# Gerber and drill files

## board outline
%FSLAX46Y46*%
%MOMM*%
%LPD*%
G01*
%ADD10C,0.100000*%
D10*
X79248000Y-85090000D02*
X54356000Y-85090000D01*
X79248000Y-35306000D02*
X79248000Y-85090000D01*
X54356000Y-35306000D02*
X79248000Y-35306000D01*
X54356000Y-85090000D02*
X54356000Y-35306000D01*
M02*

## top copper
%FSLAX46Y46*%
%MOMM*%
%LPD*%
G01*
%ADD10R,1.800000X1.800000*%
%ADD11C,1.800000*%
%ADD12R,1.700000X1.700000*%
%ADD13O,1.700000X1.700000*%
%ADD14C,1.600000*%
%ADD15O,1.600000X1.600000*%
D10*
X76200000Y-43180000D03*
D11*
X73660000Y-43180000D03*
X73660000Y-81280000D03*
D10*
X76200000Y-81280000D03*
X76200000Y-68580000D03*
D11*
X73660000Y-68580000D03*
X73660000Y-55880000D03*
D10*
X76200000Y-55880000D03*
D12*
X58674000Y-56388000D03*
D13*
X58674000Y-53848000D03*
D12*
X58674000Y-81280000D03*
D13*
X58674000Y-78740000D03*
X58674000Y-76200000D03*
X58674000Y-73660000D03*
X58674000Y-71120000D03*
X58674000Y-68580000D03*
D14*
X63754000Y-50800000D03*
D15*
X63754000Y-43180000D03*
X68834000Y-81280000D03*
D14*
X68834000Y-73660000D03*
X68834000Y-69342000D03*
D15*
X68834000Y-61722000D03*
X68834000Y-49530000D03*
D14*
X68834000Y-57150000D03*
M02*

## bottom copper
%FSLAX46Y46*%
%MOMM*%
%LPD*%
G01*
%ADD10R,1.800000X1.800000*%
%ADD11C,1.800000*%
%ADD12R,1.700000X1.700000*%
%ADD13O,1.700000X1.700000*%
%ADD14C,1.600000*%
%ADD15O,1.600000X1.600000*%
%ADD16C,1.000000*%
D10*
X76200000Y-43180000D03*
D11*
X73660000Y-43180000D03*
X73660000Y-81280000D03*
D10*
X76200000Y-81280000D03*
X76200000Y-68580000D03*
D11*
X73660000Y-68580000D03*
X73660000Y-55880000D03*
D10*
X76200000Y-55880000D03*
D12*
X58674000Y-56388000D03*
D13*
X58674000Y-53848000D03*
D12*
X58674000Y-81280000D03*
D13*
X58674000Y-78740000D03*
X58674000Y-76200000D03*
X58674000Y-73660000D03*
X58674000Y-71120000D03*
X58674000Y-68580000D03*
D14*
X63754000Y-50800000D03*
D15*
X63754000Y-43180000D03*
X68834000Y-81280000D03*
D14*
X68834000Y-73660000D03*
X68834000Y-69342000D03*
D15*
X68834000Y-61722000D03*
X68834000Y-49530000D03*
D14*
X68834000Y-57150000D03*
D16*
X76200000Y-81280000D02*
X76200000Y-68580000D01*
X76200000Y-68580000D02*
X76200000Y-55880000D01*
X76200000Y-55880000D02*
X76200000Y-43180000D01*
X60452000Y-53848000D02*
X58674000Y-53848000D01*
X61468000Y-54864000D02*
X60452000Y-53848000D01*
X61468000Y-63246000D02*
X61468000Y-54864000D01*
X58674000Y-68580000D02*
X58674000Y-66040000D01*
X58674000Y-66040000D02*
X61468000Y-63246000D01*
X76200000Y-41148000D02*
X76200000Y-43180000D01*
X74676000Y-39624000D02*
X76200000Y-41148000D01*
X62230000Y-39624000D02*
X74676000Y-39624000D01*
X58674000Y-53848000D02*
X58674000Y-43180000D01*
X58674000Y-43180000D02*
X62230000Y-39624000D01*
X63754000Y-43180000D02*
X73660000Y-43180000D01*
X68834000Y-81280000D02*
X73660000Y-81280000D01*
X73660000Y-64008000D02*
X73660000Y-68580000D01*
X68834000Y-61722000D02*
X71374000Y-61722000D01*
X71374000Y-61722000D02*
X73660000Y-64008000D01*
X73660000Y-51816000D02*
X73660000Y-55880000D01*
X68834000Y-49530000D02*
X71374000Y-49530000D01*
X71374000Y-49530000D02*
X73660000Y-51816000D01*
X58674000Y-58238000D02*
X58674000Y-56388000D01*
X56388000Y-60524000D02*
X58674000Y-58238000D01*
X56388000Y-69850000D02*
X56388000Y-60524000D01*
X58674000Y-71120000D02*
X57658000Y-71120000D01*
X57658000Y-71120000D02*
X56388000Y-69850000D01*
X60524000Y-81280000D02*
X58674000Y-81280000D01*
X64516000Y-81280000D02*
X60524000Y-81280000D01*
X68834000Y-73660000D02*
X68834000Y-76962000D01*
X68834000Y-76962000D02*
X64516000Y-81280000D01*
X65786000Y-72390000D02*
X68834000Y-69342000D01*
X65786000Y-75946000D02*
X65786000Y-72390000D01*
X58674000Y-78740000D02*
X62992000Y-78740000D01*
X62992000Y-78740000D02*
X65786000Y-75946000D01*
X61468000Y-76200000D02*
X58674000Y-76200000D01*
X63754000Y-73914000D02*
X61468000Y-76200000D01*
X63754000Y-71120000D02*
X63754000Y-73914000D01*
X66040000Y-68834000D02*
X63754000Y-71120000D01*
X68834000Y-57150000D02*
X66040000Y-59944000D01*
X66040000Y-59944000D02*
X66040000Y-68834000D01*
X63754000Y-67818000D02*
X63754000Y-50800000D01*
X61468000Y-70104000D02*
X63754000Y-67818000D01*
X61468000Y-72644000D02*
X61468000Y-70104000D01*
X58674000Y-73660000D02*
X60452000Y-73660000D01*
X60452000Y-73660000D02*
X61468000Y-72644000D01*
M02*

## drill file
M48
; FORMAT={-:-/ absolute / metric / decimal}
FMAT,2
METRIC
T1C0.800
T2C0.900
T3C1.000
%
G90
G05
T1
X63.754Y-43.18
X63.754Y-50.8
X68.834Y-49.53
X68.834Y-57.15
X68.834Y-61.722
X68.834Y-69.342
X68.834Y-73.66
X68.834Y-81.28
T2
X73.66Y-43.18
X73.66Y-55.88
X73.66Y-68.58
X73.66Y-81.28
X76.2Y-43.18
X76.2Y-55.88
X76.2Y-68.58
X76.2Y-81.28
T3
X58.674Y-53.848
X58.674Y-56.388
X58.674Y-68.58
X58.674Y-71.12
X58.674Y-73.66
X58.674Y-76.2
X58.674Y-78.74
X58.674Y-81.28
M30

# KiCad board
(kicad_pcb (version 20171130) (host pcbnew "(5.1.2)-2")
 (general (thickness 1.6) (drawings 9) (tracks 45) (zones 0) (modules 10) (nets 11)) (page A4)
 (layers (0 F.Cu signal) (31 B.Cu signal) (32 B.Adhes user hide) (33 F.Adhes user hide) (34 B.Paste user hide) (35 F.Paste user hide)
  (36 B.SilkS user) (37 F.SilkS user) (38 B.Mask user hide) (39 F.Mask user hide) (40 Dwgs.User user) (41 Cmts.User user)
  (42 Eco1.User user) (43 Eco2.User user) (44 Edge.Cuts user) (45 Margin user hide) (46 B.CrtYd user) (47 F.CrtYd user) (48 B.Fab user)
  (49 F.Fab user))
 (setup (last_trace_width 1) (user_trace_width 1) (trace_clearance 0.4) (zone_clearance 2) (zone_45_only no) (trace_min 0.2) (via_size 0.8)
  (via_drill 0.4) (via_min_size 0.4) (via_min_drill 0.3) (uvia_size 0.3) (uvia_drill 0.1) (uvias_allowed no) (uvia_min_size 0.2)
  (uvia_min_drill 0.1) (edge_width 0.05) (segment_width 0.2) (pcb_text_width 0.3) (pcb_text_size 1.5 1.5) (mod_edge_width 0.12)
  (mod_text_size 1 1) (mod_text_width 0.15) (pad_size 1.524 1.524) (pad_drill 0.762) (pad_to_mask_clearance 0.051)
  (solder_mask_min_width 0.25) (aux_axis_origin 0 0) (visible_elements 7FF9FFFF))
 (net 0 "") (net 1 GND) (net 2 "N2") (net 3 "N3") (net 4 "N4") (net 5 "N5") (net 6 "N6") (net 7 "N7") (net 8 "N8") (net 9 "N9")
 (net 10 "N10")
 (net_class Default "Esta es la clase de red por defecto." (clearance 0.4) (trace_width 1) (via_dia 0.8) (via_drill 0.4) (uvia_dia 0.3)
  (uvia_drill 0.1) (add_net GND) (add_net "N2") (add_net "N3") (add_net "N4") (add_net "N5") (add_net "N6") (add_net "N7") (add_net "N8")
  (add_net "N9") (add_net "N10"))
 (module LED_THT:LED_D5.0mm (layer F.Cu) (at 76.2 43.18 180)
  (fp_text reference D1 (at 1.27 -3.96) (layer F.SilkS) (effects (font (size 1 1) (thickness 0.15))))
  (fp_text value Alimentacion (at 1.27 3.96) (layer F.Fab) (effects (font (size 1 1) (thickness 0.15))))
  (pad 1 thru_hole rect (at 0 0 180) (size 1.8 1.8) (drill 0.9) (layers *.Cu *.Mask) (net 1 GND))
  (pad 2 thru_hole circle (at 2.54 0 180) (size 1.8 1.8) (drill 0.9) (layers *.Cu *.Mask) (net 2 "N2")))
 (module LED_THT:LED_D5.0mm (layer F.Cu) (at 76.2 81.28 180)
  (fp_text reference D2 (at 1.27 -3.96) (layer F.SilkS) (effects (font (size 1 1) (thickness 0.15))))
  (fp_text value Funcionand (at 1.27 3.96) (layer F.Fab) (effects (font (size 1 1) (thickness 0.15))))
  (pad 2 thru_hole circle (at 2.54 0 180) (size 1.8 1.8) (drill 0.9) (layers *.Cu *.Mask) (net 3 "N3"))
  (pad 1 thru_hole rect (at 0 0 180) (size 1.8 1.8) (drill 0.9) (layers *.Cu *.Mask) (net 1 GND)))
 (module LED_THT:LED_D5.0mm (layer F.Cu) (at 76.2 68.58 180)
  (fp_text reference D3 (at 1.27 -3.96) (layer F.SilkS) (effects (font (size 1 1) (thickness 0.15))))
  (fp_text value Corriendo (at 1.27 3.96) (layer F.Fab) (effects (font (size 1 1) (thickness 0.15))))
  (pad 1 thru_hole rect (at 0 0 180) (size 1.8 1.8) (drill 0.9) (layers *.Cu *.Mask) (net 1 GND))
  (pad 2 thru_hole circle (at 2.54 0 180) (size 1.8 1.8) (drill 0.9) (layers *.Cu *.Mask) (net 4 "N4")))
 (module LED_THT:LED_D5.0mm (layer F.Cu) (at 76.2 55.88 180)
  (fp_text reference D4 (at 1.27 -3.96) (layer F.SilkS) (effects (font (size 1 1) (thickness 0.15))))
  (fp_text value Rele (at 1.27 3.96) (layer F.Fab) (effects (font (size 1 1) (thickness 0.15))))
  (pad 2 thru_hole circle (at 2.54 0 180) (size 1.8 1.8) (drill 0.9) (layers *.Cu *.Mask) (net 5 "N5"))
  (pad 1 thru_hole rect (at 0 0 180) (size 1.8 1.8) (drill 0.9) (layers *.Cu *.Mask) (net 1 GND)))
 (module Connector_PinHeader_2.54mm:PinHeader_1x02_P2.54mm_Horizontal (layer F.Cu) (at 58.674 56.388 180)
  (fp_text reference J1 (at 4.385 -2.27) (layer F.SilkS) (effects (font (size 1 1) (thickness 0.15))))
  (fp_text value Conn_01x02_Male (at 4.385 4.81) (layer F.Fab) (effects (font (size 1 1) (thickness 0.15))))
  (pad 1 thru_hole rect (at 0 0 180) (size 1.7 1.7) (drill 1) (layers *.Cu *.Mask) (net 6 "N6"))
  (pad 2 thru_hole oval (at 0 2.54 180) (size 1.7 1.7) (drill 1) (layers *.Cu *.Mask) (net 1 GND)))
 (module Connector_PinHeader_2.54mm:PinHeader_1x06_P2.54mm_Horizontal (layer F.Cu) (at 58.674 81.28 180)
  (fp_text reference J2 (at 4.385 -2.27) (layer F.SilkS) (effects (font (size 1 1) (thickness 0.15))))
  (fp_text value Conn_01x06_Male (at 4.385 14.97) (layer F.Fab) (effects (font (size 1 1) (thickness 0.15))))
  (pad 1 thru_hole rect (at 0 0 180) (size 1.7 1.7) (drill 1) (layers *.Cu *.Mask) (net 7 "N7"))
  (pad 2 thru_hole oval (at 0 2.54 180) (size 1.7 1.7) (drill 1) (layers *.Cu *.Mask) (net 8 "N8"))
  (pad 3 thru_hole oval (at 0 5.08 180) (size 1.7 1.7) (drill 1) (layers *.Cu *.Mask) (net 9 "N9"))
  (pad 4 thru_hole oval (at 0 7.62 180) (size 1.7 1.7) (drill 1) (layers *.Cu *.Mask) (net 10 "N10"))
  (pad 5 thru_hole oval (at 0 10.16 180) (size 1.7 1.7) (drill 1) (layers *.Cu *.Mask) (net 6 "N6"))
  (pad 6 thru_hole oval (at 0 12.7 180) (size 1.7 1.7) (drill 1) (layers *.Cu *.Mask) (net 1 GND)))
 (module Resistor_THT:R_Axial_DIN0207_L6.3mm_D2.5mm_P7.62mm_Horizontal (layer F.Cu) (at 63.754 50.8 90)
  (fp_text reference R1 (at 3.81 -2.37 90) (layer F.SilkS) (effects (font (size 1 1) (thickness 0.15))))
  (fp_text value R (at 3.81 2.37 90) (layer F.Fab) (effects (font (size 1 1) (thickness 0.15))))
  (pad 1 thru_hole circle (at 0 0 90) (size 1.6 1.6) (drill 0.8) (layers *.Cu *.Mask) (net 10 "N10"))
  (pad 2 thru_hole oval (at 7.62 0 90) (size 1.6 1.6) (drill 0.8) (layers *.Cu *.Mask) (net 2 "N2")))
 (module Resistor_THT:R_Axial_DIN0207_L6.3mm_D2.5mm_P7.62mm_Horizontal (layer F.Cu) (at 68.834 73.66 270)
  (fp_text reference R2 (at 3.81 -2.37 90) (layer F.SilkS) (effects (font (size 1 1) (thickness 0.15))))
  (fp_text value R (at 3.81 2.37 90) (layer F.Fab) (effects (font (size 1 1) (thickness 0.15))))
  (pad 2 thru_hole oval (at 7.62 0 270) (size 1.6 1.6) (drill 0.8) (layers *.Cu *.Mask) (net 3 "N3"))
  (pad 1 thru_hole circle (at 0 0 270) (size 1.6 1.6) (drill 0.8) (layers *.Cu *.Mask) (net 7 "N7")))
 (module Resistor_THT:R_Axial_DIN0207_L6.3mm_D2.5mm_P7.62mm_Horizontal (layer F.Cu) (at 68.834 69.342 90)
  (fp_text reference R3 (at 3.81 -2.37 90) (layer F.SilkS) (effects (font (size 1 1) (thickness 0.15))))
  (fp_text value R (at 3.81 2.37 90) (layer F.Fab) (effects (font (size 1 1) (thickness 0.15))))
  (pad 1 thru_hole circle (at 0 0 90) (size 1.6 1.6) (drill 0.8) (layers *.Cu *.Mask) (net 8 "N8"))
  (pad 2 thru_hole oval (at 7.62 0 90) (size 1.6 1.6) (drill 0.8) (layers *.Cu *.Mask) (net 4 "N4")))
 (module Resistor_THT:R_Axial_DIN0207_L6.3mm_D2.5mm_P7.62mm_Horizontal (layer F.Cu) (at 68.834 57.15 90)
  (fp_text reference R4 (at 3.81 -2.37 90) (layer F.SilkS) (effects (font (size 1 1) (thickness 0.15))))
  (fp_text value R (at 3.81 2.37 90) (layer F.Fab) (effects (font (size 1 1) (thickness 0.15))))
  (pad 2 thru_hole oval (at 7.62 0 90) (size 1.6 1.6) (drill 0.8) (layers *.Cu *.Mask) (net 5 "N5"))
  (pad 1 thru_hole circle (at 0 0 90) (size 1.6 1.6) (drill 0.8) (layers *.Cu *.Mask) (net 9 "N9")))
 (gr_line (start 79.248 85.09) (end 54.356 85.09) (layer Edge.Cuts) (width 0.1))
 (gr_line (start 79.248 35.306) (end 79.248 85.09) (layer Edge.Cuts) (width 0.1))
 (gr_line (start 54.356 35.306) (end 79.248 35.306) (layer Edge.Cuts) (width 0.1))
 (gr_line (start 54.356 85.09) (end 54.356 35.306) (layer Edge.Cuts) (width 0.1))
 (segment (start 76.2 81.28) (end 76.2 68.58) (width 1) (layer B.Cu) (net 1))
 (segment (start 76.2 68.58) (end 76.2 55.88) (width 1) (layer B.Cu) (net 1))
 (segment (start 76.2 55.88) (end 76.2 43.18) (width 1) (layer B.Cu) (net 1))
 (segment (start 60.452 53.848) (end 58.674 53.848) (width 1) (layer B.Cu) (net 1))
 (segment (start 61.468 54.864) (end 60.452 53.848) (width 1) (layer B.Cu) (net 1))
 (segment (start 61.468 63.246) (end 61.468 54.864) (width 1) (layer B.Cu) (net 1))
 (segment (start 58.674 68.58) (end 58.674 66.04) (width 1) (layer B.Cu) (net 1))
 (segment (start 58.674 66.04) (end 61.468 63.246) (width 1) (layer B.Cu) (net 1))
 (segment (start 76.2 41.148) (end 76.2 43.18) (width 1) (layer B.Cu) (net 1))
 (segment (start 74.676 39.624) (end 76.2 41.148) (width 1) (layer B.Cu) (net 1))
 (segment (start 62.23 39.624) (end 74.676 39.624) (width 1) (layer B.Cu) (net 1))
 (segment (start 58.674 53.848) (end 58.674 43.18) (width 1) (layer B.Cu) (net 1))
 (segment (start 58.674 43.18) (end 62.23 39.624) (width 1) (layer B.Cu) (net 1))
 (segment (start 63.754 43.18) (end 73.66 43.18) (width 1) (layer B.Cu) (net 2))
 (segment (start 68.834 81.28) (end 73.66 81.28) (width 1) (layer B.Cu) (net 3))
 (segment (start 73.66 64.008) (end 73.66 68.58) (width 1) (layer B.Cu) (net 4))
 (segment (start 68.834 61.722) (end 71.374 61.722) (width 1) (layer B.Cu) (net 4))
 (segment (start 71.374 61.722) (end 73.66 64.008) (width 1) (layer B.Cu) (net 4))
 (segment (start 73.66 51.816) (end 73.66 55.88) (width 1) (layer B.Cu) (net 5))
 (segment (start 68.834 49.53) (end 71.374 49.53) (width 1) (layer B.Cu) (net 5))
 (segment (start 71.374 49.53) (end 73.66 51.816) (width 1) (layer B.Cu) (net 5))
 (segment (start 58.674 58.238) (end 58.674 56.388) (width 1) (layer B.Cu) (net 6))
 (segment (start 56.388 60.524) (end 58.674 58.238) (width 1) (layer B.Cu) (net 6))
 (segment (start 56.388 69.85) (end 56.388 60.524) (width 1) (layer B.Cu) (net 6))
 (segment (start 58.674 71.12) (end 57.658 71.12) (width 1) (layer B.Cu) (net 6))
 (segment (start 57.658 71.12) (end 56.388 69.85) (width 1) (layer B.Cu) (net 6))
 (segment (start 60.524 81.28) (end 58.674 81.28) (width 1) (layer B.Cu) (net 7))
 (segment (start 64.516 81.28) (end 60.524 81.28) (width 1) (layer B.Cu) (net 7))
 (segment (start 68.834 73.66) (end 68.834 76.962) (width 1) (layer B.Cu) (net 7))
 (segment (start 68.834 76.962) (end 64.516 81.28) (width 1) (layer B.Cu) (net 7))
 (segment (start 65.786 72.39) (end 68.834 69.342) (width 1) (layer B.Cu) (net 8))
 (segment (start 65.786 75.946) (end 65.786 72.39) (width 1) (layer B.Cu) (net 8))
 (segment (start 58.674 78.74) (end 62.992 78.74) (width 1) (layer B.Cu) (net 8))
 (segment (start 62.992 78.74) (end 65.786 75.946) (width 1) (layer B.Cu) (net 8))
 (segment (start 61.468 76.2) (end 58.674 76.2) (width 1) (layer B.Cu) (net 9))
 (segment (start 63.754 73.914) (end 61.468 76.2) (width 1) (layer B.Cu) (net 9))
 (segment (start 63.754 71.12) (end 63.754 73.914) (width 1) (layer B.Cu) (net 9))
 (segment (start 66.04 68.834) (end 63.754 71.12) (width 1) (layer B.Cu) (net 9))
 (segment (start 68.834 57.15) (end 66.04 59.944) (width 1) (layer B.Cu) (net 9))
 (segment (start 66.04 59.944) (end 66.04 68.834) (width 1) (layer B.Cu) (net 9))
 (segment (start 63.754 67.818) (end 63.754 50.8) (width 1) (layer B.Cu) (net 10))
 (segment (start 61.468 70.104) (end 63.754 67.818) (width 1) (layer B.Cu) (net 10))
 (segment (start 61.468 72.644) (end 61.468 70.104) (width 1) (layer B.Cu) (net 10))
 (segment (start 58.674 73.66) (end 60.452 73.66) (width 1) (layer B.Cu) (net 10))
 (segment (start 60.452 73.66) (end 61.468 72.644) (width 1) (layer B.Cu) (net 10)))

